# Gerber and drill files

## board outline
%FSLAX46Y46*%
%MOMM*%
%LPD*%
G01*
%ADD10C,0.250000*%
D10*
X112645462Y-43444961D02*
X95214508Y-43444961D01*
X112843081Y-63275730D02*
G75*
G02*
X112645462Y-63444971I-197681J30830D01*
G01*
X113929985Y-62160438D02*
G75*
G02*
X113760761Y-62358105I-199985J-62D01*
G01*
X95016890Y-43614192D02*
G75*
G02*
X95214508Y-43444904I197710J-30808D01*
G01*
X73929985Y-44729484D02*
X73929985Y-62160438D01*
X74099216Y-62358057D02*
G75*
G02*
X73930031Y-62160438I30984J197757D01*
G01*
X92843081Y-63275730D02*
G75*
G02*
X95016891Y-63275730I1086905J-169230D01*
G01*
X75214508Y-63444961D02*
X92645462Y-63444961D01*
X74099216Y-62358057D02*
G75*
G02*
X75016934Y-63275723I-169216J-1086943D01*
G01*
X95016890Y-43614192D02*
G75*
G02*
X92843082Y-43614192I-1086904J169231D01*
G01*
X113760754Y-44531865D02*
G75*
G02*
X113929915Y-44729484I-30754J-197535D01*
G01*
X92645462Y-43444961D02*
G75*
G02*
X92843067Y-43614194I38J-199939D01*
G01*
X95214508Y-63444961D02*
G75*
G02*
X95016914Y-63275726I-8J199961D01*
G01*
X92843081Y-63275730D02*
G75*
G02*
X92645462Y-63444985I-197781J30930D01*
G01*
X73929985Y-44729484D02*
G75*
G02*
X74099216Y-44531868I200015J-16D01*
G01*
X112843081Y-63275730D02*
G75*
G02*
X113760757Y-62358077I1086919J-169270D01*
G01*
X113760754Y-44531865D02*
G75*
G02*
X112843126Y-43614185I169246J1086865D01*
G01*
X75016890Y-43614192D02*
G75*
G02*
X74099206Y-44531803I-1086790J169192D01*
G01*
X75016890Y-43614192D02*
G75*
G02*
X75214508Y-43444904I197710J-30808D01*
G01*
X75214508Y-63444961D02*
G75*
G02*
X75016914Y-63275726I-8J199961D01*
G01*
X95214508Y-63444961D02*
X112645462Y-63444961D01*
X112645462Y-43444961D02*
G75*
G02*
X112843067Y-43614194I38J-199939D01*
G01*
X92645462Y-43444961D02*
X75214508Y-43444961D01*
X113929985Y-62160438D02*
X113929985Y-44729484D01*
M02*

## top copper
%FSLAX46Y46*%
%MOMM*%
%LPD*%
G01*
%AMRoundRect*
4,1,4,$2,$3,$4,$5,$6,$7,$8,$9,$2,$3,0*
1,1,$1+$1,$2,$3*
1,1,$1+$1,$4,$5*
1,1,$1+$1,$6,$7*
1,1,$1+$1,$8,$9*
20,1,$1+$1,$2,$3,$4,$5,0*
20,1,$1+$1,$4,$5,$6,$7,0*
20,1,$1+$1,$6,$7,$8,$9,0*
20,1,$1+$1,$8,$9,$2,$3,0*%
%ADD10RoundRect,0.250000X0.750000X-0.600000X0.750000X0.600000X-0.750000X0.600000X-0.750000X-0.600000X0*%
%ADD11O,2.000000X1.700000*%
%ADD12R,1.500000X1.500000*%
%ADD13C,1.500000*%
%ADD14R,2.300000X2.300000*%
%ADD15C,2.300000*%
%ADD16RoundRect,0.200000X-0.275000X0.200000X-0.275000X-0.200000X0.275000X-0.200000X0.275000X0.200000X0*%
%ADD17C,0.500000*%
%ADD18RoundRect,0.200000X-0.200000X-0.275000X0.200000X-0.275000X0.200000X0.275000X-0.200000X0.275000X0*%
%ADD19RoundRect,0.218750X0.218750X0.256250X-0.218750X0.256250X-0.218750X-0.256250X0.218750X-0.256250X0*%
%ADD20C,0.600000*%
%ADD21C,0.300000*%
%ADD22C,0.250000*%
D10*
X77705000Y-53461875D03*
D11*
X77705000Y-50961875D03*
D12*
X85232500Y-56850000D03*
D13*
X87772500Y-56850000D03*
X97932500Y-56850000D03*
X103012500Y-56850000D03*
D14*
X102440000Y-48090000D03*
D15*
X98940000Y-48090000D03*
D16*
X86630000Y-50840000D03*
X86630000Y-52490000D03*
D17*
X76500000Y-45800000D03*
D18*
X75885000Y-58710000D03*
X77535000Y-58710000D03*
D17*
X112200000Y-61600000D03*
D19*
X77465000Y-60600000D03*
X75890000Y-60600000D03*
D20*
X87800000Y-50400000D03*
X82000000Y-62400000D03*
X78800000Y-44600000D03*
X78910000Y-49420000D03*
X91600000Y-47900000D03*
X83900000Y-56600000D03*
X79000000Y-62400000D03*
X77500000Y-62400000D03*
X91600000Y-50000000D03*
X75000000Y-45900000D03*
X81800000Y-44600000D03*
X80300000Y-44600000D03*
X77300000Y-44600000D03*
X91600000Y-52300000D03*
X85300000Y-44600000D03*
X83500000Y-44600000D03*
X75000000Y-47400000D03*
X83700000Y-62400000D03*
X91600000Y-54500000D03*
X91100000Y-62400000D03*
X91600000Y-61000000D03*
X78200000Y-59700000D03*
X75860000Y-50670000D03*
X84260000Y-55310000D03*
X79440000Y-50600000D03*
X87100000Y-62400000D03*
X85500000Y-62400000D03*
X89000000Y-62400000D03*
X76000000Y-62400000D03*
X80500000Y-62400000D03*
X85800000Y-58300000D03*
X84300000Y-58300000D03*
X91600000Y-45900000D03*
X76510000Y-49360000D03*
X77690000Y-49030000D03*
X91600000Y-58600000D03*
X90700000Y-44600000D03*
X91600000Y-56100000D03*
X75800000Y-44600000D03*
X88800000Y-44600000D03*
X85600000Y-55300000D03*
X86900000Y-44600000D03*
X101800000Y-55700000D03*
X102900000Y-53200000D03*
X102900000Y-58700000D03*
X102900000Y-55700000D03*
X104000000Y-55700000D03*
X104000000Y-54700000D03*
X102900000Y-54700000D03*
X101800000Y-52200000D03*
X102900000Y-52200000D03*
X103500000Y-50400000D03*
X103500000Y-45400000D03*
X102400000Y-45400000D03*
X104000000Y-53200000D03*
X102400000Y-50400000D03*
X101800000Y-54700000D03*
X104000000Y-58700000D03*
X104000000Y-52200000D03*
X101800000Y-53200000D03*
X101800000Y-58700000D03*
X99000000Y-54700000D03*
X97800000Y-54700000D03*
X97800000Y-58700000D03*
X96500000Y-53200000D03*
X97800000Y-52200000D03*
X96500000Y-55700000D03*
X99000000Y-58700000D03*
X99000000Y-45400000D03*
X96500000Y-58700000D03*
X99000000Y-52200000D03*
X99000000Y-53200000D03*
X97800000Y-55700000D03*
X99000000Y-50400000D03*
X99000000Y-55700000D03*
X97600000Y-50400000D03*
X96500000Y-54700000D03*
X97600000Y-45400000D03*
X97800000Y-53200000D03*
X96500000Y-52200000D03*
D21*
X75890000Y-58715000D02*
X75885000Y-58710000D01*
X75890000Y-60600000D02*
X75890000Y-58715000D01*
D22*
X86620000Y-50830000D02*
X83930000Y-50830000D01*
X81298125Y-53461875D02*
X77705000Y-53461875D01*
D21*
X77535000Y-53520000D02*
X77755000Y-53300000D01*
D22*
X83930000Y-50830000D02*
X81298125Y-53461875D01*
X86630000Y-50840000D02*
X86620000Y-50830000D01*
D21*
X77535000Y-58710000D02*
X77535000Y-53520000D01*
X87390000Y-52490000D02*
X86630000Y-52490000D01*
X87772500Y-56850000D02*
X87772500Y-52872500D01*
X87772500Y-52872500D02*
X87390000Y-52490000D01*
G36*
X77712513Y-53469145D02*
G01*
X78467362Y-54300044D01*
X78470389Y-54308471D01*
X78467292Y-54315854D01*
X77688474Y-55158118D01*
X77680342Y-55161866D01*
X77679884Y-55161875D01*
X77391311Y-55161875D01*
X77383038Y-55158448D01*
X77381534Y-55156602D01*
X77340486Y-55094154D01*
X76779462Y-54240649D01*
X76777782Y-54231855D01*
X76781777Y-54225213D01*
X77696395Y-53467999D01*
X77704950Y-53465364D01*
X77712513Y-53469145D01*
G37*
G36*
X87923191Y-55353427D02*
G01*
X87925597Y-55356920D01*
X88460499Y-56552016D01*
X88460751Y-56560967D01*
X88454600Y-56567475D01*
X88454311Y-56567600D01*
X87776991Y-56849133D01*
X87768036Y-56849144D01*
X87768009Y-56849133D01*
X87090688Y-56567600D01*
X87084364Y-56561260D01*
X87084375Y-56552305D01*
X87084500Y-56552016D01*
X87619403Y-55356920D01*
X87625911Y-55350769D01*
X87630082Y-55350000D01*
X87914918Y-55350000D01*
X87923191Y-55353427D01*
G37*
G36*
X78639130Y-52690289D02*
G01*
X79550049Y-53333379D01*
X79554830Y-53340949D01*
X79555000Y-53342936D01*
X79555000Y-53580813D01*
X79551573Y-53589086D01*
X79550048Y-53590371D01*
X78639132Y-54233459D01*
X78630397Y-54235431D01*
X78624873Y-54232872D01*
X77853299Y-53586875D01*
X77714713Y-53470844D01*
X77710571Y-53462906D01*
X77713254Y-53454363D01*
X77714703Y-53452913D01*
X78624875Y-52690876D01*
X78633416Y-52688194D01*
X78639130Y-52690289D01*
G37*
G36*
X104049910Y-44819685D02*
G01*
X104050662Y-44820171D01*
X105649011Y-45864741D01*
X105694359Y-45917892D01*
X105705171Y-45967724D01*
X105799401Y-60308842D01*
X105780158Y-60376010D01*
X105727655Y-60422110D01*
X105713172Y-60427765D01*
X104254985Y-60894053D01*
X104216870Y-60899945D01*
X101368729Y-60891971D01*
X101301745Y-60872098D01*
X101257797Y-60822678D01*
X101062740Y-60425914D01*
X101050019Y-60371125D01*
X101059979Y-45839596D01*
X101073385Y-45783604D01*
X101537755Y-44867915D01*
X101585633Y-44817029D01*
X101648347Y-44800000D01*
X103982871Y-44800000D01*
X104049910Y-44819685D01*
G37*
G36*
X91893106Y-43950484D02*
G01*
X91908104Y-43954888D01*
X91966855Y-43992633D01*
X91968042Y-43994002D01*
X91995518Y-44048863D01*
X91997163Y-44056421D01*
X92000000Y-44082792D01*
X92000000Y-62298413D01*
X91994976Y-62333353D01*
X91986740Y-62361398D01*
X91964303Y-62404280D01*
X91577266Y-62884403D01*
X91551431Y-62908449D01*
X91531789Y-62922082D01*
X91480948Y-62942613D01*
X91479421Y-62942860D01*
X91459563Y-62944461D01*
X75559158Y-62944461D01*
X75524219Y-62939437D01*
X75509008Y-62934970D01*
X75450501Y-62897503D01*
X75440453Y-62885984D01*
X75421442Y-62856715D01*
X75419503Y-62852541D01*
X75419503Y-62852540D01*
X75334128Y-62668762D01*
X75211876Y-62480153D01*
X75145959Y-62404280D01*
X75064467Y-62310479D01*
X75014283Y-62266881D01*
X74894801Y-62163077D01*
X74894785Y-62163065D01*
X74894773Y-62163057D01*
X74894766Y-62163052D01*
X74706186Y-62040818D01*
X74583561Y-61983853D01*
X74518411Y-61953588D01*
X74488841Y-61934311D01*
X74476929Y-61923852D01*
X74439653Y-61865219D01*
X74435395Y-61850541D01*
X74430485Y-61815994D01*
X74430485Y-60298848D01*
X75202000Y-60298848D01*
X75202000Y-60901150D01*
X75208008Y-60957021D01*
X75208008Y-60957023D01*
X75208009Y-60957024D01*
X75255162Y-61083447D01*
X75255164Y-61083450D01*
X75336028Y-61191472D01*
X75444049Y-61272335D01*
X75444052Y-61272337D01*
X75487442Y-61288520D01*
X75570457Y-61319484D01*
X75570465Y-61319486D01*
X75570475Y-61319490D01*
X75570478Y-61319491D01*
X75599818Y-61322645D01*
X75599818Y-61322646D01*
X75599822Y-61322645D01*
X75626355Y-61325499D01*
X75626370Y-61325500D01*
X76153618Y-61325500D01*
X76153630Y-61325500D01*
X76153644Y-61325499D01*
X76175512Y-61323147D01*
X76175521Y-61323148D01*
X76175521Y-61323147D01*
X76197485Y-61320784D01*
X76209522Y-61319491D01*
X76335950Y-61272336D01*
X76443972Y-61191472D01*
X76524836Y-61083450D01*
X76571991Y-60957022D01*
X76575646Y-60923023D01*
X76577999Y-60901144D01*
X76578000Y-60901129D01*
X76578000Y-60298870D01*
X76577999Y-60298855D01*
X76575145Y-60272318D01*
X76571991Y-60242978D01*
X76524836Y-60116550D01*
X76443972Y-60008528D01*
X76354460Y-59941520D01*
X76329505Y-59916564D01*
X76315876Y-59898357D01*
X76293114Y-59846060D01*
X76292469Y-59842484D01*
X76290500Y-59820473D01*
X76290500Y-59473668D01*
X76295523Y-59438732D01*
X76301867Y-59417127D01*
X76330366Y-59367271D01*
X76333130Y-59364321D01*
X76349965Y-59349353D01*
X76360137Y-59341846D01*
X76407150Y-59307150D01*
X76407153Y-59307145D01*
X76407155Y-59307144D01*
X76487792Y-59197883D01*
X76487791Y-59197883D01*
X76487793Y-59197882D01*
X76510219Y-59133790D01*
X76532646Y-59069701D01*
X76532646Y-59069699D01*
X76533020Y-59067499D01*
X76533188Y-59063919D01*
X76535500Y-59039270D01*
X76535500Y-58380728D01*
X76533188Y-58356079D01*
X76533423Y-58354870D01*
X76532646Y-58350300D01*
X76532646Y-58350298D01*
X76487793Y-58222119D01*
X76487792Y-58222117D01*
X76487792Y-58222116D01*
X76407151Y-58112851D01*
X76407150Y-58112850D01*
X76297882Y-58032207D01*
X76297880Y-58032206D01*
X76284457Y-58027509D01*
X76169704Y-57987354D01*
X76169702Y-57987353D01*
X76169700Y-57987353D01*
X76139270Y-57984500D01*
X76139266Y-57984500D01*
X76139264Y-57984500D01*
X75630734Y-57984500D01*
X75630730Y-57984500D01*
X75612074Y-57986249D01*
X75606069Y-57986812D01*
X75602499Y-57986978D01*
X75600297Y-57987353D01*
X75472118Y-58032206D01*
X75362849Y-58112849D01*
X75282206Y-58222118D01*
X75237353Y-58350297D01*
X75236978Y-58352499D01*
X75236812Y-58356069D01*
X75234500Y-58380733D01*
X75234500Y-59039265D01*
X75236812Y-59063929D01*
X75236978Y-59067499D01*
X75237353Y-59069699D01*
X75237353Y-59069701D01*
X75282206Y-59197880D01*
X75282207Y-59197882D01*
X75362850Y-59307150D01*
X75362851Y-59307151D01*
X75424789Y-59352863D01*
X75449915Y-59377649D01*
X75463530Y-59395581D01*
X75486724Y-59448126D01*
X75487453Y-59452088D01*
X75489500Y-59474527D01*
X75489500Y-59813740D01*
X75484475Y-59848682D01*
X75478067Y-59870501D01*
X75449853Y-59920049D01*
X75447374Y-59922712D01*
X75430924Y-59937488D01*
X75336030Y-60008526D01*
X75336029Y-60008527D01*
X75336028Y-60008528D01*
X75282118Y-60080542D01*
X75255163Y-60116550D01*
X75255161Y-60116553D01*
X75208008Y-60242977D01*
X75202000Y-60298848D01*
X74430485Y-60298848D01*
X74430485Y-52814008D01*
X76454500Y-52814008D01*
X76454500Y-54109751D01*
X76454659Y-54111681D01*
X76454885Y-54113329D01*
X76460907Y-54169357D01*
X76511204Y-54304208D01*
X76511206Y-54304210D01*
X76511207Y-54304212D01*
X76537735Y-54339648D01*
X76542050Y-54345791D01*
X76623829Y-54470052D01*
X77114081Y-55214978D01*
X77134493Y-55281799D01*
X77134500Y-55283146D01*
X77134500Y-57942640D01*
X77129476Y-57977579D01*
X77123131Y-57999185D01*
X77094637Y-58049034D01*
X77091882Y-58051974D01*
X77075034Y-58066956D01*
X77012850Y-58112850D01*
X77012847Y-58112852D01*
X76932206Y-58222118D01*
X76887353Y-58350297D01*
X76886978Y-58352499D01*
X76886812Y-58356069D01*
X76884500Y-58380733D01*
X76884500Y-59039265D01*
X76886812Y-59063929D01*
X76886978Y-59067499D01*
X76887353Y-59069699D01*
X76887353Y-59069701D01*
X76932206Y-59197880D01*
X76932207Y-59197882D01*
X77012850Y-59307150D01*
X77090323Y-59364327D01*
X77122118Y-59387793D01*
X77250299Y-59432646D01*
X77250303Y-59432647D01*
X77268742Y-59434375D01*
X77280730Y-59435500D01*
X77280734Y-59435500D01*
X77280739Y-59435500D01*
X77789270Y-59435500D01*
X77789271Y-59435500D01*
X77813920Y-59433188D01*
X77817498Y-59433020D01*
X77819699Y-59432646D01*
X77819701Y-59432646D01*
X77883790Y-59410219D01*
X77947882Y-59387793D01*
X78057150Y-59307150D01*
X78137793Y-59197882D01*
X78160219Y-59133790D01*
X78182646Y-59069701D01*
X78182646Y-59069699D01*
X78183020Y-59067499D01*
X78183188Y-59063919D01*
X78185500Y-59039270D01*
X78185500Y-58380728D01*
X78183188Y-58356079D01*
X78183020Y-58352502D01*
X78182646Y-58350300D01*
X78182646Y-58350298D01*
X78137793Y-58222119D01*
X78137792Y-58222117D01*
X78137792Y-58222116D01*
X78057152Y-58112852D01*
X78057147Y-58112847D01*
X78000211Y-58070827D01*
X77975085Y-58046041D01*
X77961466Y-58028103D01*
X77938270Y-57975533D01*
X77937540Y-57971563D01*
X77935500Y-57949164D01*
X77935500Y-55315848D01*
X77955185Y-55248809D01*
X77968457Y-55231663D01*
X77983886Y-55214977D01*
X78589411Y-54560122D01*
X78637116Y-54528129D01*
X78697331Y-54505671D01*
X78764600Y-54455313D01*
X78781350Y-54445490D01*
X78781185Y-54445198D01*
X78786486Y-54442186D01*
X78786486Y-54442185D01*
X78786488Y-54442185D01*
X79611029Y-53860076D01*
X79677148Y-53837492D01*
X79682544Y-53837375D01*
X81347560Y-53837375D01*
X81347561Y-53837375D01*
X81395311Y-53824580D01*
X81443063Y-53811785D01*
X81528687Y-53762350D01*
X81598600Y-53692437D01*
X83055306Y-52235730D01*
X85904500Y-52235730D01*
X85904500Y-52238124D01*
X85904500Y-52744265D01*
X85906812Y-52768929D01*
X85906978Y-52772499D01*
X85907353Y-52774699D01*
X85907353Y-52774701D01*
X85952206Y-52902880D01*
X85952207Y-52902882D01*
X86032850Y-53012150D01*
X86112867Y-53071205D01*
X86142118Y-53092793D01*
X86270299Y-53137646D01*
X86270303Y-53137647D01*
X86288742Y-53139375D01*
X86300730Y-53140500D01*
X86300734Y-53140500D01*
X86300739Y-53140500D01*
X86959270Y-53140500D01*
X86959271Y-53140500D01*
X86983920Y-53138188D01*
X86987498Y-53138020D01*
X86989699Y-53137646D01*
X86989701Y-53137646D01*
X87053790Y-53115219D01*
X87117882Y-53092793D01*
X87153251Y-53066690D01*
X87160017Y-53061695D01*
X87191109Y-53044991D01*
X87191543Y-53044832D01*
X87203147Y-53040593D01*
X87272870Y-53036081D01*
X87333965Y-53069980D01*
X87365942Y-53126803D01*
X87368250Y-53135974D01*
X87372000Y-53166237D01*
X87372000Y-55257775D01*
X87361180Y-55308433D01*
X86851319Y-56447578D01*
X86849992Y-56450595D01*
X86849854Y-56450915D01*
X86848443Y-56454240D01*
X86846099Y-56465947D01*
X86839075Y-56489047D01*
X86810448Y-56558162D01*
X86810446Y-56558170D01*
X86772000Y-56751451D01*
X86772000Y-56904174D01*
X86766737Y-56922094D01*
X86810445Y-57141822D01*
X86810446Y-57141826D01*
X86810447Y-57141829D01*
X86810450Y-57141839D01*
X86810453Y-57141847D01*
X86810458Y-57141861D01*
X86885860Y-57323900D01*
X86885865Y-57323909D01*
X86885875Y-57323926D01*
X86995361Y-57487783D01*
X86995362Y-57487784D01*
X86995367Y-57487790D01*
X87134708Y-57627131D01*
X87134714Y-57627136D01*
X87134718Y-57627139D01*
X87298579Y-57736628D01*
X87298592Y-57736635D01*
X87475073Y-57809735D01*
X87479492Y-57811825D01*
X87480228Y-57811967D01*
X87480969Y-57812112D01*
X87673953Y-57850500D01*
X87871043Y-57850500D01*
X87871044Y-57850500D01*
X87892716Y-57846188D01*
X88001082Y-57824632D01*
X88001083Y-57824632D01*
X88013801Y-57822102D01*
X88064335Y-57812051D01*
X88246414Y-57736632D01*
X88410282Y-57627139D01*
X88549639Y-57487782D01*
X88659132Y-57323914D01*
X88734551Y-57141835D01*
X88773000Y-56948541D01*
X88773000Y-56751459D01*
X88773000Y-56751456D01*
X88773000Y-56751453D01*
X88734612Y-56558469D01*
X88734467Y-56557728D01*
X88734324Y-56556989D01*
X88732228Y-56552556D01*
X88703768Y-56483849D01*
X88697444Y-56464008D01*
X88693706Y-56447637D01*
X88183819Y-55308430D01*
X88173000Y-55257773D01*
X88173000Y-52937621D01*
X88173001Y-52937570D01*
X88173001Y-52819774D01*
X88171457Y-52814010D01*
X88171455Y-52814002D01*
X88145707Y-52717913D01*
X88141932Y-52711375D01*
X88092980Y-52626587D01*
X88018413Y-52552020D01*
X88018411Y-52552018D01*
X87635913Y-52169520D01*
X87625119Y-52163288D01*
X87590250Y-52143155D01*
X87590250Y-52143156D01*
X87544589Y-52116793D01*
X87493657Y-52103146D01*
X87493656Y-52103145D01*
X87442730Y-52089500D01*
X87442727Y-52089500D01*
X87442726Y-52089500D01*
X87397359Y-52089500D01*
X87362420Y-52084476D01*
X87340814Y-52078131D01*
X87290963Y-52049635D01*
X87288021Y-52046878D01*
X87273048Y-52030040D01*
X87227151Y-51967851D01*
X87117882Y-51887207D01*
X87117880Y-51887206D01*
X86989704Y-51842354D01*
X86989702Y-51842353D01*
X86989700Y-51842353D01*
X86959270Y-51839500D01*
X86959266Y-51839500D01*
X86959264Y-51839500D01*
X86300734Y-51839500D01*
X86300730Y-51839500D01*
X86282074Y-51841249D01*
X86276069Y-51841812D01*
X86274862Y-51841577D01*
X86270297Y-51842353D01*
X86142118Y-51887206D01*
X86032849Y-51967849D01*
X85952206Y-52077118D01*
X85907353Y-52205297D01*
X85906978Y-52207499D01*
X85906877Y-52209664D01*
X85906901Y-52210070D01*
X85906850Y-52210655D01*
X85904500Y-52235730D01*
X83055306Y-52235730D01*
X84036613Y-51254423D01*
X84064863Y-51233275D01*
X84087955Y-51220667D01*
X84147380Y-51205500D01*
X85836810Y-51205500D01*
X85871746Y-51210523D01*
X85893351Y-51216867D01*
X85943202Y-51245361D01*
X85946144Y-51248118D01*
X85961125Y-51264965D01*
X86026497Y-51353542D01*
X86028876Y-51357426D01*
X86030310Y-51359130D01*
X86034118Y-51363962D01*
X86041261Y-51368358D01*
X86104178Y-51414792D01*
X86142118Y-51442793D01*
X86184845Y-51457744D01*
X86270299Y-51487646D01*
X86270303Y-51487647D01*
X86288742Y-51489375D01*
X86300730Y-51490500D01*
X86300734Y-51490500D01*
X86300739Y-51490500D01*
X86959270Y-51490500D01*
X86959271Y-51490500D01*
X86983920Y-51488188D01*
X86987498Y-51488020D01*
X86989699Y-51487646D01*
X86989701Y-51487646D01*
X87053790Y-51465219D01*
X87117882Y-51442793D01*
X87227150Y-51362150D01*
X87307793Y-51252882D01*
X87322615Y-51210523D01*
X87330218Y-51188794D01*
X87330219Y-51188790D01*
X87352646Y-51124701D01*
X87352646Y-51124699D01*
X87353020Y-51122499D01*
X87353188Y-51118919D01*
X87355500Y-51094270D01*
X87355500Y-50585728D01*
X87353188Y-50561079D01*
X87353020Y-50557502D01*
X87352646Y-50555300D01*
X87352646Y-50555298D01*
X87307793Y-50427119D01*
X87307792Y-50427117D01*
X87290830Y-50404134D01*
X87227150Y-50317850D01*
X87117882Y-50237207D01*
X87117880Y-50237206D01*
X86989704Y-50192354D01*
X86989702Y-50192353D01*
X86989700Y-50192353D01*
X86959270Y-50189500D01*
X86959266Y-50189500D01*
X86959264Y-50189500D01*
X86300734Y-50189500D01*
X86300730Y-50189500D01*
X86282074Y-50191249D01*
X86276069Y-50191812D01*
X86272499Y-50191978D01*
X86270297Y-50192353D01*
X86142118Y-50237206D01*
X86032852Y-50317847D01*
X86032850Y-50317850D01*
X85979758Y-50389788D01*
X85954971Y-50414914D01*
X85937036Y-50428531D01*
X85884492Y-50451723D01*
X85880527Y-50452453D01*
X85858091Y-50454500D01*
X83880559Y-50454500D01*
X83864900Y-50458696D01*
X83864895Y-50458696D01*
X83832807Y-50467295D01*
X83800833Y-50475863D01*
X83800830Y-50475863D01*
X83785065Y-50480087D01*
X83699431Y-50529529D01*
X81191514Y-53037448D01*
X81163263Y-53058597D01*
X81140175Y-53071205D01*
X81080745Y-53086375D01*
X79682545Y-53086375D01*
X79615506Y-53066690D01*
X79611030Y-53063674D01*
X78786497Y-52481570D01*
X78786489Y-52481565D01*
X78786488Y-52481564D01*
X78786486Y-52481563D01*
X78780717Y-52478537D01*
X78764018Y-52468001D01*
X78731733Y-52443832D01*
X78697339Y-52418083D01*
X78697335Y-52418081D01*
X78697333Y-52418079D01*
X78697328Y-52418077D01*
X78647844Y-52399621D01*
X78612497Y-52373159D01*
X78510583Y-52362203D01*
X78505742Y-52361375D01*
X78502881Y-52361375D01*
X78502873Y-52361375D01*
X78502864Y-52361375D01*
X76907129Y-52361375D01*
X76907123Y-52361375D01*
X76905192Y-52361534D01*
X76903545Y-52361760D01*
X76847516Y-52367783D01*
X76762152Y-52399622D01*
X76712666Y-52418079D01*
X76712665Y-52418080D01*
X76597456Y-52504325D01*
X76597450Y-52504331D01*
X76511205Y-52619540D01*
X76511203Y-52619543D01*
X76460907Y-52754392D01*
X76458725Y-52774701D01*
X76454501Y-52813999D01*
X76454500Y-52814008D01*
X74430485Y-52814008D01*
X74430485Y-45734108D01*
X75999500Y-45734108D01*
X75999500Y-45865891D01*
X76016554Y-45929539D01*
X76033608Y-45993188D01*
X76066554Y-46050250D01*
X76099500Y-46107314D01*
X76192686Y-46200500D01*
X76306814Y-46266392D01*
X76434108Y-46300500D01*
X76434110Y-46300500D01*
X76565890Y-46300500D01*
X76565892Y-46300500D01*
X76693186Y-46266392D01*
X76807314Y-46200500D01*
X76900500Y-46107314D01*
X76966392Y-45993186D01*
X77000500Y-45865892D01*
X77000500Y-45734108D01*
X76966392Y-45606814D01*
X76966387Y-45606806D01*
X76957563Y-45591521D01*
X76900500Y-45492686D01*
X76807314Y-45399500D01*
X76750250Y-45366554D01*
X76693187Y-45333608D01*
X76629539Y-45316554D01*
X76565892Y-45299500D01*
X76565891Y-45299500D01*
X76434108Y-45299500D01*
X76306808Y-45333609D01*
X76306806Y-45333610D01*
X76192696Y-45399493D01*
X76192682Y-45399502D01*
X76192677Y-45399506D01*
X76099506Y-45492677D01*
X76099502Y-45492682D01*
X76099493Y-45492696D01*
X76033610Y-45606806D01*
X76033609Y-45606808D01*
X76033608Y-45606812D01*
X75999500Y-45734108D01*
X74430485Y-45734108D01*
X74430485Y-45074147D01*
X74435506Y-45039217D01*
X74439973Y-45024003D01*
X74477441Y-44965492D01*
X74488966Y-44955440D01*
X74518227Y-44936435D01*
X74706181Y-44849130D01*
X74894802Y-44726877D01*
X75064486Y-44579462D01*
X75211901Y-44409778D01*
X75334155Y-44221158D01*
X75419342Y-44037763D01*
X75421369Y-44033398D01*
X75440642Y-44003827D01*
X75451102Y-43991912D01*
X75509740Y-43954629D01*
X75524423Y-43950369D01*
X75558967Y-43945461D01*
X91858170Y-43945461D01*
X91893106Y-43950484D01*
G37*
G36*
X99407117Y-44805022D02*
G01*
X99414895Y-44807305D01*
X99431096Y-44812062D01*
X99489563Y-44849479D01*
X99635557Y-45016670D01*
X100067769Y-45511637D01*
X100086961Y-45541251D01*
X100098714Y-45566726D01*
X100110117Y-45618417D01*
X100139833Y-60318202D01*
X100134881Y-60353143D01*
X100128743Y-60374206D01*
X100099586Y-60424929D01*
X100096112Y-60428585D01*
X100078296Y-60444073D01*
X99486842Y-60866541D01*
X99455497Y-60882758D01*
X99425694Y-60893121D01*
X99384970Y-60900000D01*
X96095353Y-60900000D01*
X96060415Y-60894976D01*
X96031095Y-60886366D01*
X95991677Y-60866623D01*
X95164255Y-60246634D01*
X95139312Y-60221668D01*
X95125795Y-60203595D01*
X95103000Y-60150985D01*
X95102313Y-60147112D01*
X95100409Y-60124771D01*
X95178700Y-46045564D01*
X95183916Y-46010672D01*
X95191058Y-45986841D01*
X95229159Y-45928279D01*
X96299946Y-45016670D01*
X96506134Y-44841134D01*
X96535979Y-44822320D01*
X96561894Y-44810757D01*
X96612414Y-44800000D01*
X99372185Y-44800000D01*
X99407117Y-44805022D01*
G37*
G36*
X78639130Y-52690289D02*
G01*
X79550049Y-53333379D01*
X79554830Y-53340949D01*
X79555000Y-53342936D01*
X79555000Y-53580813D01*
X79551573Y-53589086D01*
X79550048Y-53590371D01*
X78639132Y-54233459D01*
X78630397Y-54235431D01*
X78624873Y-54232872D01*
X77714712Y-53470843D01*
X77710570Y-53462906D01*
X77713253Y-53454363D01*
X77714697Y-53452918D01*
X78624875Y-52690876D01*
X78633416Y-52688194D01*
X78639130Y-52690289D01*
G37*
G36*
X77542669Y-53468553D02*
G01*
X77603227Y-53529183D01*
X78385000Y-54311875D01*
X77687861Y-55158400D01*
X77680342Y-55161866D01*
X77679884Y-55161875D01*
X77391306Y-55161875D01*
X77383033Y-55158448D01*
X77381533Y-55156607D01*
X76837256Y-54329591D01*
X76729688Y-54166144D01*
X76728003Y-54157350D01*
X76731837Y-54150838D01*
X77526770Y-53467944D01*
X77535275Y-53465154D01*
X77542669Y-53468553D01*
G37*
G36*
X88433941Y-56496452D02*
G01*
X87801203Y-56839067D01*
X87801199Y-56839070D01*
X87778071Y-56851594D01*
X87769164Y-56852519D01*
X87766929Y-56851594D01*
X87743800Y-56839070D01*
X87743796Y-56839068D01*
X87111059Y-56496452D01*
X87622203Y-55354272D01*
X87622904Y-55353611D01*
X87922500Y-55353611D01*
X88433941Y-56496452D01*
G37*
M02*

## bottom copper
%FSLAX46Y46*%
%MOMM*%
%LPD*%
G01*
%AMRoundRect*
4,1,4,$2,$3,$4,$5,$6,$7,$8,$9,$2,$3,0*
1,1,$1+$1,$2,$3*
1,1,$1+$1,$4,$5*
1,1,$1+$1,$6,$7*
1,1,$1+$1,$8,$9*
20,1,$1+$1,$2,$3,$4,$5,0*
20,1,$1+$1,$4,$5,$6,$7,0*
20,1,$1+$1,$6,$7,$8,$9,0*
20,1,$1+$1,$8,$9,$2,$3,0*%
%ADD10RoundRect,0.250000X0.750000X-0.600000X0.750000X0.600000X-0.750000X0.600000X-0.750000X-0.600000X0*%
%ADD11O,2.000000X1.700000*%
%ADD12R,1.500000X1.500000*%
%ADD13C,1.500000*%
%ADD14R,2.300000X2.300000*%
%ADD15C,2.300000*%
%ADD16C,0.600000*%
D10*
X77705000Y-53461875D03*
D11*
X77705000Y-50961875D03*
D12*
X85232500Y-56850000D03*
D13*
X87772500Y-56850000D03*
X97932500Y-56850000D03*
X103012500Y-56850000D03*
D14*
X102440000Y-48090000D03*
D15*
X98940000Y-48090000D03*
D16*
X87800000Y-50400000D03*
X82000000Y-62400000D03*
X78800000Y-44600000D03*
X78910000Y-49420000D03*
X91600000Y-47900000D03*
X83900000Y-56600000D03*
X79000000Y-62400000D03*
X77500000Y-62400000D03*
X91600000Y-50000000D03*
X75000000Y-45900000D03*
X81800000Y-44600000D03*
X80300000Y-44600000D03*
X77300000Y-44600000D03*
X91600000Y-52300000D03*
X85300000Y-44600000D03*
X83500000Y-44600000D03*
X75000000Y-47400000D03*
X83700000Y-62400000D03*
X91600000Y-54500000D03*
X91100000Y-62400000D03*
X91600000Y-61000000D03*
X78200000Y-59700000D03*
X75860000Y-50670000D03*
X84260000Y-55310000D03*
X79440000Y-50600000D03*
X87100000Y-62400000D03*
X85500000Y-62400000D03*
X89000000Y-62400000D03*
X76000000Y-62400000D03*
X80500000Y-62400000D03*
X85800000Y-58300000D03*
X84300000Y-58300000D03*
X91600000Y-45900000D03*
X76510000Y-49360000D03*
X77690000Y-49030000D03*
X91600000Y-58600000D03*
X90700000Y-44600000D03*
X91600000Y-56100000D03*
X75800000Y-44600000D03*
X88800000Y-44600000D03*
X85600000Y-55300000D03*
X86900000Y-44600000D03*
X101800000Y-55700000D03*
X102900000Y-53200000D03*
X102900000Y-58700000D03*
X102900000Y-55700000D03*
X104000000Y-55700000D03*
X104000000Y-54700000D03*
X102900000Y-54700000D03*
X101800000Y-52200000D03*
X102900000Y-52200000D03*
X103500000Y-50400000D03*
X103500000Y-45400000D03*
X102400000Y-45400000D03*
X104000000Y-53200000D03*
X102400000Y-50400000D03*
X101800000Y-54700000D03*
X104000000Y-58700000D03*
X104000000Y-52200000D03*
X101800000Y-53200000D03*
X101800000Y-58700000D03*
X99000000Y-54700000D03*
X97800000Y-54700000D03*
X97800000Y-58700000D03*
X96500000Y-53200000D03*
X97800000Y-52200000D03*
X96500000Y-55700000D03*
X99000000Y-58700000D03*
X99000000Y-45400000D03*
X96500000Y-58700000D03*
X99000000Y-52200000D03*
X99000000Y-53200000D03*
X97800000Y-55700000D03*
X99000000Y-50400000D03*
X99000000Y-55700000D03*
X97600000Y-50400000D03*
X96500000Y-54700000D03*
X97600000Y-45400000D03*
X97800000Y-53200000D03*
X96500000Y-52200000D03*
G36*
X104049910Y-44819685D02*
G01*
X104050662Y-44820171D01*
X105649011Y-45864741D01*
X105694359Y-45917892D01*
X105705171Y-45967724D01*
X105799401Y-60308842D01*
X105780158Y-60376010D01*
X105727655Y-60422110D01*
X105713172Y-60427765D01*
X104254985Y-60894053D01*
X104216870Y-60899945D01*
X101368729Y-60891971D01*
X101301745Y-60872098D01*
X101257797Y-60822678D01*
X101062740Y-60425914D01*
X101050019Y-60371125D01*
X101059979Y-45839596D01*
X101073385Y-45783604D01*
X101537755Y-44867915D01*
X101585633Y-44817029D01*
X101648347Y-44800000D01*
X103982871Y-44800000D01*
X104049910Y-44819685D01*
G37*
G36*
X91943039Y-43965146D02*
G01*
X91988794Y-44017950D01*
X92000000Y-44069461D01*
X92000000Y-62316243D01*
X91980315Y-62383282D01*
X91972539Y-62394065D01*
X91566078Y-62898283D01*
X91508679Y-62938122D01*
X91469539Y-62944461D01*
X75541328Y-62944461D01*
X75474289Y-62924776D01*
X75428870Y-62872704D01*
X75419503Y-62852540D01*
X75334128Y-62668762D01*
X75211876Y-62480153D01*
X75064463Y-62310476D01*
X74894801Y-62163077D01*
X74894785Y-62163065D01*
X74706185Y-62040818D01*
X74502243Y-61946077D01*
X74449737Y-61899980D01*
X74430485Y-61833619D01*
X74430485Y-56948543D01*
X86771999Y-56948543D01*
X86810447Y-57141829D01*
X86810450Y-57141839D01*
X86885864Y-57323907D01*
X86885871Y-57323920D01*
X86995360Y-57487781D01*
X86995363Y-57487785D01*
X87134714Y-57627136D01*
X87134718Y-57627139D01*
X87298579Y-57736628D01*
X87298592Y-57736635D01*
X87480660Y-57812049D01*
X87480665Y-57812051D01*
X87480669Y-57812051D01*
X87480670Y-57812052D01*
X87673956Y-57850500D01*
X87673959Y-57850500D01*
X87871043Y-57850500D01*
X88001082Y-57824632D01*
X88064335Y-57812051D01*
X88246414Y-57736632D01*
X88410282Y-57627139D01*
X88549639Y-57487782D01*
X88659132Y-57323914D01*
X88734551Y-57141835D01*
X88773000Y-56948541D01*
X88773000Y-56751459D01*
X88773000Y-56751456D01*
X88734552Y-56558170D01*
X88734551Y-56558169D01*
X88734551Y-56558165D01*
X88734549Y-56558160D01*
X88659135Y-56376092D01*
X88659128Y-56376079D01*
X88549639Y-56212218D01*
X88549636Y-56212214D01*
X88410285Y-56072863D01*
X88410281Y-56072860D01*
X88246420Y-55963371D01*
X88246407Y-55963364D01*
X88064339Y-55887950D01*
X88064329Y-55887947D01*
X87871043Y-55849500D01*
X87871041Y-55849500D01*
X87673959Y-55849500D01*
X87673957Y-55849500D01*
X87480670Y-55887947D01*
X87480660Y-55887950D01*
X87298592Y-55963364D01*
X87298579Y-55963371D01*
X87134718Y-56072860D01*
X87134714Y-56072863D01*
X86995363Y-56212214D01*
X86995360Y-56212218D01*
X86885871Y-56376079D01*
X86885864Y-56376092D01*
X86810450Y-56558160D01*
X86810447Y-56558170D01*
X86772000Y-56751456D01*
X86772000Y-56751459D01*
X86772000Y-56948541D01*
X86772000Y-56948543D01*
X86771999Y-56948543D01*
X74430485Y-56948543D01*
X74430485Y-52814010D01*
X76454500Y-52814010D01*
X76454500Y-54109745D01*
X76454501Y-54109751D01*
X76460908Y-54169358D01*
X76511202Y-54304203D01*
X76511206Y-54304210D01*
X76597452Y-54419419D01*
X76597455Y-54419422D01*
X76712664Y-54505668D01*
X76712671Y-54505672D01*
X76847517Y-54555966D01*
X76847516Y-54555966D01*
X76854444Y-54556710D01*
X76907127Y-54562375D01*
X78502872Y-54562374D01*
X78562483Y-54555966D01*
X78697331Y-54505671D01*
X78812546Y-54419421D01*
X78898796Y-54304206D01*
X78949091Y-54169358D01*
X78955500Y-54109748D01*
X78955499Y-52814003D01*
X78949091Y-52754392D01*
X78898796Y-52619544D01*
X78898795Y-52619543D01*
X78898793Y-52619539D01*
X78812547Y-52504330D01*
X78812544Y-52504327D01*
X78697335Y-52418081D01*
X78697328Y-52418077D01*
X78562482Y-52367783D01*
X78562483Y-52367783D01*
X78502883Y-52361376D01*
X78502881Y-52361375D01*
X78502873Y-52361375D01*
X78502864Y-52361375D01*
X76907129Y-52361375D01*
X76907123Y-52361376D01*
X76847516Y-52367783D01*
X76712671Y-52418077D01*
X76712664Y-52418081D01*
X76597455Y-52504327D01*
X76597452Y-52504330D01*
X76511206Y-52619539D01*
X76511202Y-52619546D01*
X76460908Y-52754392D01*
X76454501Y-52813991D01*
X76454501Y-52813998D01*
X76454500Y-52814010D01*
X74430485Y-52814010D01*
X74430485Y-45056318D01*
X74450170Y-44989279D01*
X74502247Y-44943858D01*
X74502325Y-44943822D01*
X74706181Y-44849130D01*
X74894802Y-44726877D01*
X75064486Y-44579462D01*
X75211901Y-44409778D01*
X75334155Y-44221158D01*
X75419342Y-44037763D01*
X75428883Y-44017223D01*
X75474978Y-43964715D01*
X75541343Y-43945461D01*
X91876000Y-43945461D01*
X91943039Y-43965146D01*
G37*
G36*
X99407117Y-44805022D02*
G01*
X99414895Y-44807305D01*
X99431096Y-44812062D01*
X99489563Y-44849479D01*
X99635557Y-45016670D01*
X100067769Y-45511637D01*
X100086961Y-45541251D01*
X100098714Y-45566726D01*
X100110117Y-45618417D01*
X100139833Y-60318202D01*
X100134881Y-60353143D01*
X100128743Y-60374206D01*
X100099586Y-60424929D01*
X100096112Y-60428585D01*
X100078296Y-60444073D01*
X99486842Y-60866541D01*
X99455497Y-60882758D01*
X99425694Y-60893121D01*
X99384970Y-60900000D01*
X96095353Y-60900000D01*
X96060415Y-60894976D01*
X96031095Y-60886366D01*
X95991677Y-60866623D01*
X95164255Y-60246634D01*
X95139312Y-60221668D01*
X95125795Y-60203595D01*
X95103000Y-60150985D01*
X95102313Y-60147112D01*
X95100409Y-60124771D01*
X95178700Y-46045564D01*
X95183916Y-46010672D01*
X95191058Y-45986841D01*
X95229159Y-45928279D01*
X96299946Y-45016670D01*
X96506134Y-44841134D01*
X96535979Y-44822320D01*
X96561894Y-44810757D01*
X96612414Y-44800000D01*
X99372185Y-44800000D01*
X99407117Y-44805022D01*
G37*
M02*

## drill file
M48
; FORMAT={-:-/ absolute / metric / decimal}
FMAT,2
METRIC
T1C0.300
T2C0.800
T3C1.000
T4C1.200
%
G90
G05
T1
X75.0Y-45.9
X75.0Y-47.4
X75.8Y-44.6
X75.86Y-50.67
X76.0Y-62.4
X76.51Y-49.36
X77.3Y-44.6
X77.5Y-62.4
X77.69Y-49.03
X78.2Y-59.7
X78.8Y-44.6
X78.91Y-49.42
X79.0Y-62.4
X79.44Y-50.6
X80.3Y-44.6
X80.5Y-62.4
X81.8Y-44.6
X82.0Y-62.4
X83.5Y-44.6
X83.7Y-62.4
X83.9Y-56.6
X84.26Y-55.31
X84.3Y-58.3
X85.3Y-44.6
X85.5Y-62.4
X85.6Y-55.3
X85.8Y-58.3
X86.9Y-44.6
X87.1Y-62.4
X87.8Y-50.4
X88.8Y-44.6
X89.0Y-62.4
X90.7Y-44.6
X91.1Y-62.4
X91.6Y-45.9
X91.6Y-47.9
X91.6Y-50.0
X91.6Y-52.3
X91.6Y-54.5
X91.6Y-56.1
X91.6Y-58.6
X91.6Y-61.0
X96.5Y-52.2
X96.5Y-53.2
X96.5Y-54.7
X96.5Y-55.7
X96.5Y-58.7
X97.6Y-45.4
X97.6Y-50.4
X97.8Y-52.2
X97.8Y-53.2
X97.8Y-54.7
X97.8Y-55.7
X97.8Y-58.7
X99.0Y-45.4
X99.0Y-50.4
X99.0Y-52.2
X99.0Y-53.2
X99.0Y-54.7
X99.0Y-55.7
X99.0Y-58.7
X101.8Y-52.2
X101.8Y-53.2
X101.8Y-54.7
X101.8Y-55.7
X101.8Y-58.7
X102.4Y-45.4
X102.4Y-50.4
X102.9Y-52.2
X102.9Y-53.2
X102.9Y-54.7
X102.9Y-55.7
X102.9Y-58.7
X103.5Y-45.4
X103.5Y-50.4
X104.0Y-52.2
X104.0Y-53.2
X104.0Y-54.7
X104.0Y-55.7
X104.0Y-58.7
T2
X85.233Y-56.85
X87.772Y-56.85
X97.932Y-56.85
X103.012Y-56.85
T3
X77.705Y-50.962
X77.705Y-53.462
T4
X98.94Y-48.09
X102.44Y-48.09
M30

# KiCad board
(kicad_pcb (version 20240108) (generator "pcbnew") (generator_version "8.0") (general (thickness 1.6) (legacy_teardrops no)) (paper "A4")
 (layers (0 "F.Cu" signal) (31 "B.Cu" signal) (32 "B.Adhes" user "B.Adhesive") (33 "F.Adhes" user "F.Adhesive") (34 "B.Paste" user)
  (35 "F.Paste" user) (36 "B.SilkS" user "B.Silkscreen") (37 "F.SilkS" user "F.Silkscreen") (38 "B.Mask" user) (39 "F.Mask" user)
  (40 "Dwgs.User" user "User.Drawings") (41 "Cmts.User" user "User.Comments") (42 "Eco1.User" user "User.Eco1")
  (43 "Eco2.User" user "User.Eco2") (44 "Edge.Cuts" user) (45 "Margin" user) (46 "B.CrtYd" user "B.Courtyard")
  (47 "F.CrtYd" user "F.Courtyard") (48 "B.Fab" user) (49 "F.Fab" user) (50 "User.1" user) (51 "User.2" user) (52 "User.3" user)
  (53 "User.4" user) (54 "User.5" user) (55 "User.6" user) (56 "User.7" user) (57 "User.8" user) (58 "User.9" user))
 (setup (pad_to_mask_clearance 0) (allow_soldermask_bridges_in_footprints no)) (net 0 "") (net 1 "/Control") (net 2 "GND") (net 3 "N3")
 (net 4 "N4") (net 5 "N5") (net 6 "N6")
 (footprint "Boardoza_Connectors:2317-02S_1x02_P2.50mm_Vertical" (layer "F.Cu") (at 77.655 52.301875 90)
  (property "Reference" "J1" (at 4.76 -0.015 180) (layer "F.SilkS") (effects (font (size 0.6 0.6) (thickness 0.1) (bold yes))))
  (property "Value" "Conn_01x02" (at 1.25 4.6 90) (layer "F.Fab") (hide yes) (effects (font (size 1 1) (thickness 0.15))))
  (pad "1" thru_hole roundrect (at -1.16 0.05 90) (size 1.7 2) (drill 1) (layers "*.Cu" "*.Mask") (remove_unused_layers no)
   (roundrect_rratio 0.1470588235) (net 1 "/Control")
   (teardrops (best_length_ratio 0.5) (max_length 1) (best_width_ratio 1) (max_width 2) (curve_points 0) (filter_ratio 0.9) (enabled yes)
    (allow_two_segments yes) (prefer_zone_connections yes)))
  (pad "2" thru_hole oval (at 1.34 0.05 90) (size 1.7 2) (drill 1) (layers "*.Cu" "*.Mask") (remove_unused_layers no) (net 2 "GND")
   (teardrops (best_length_ratio 0.5) (max_length 1) (best_width_ratio 1) (max_width 2) (curve_points 0) (filter_ratio 0.9) (enabled yes)
    (allow_two_segments yes) (prefer_zone_connections yes))))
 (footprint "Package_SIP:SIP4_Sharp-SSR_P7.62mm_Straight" (layer "F.Cu") (at 103.0125 57.85 180)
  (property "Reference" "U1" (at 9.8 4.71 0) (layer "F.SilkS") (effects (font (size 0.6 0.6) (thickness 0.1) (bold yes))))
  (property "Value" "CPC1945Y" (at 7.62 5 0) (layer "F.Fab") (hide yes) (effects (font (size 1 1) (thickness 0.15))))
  (pad "1" thru_hole rect (at 17.78 1 180) (size 1.5 1.5) (drill 0.8) (layers "*.Cu" "*.Mask") (remove_unused_layers no) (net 2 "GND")
   (teardrops (best_length_ratio 0.5) (max_length 1) (best_width_ratio 1) (max_width 2) (curve_points 0) (filter_ratio 0.9) (enabled yes)
    (allow_two_segments yes) (prefer_zone_connections yes)))
  (pad "2" thru_hole circle (at 15.24 1 180) (size 1.5 1.5) (drill 0.8) (layers "*.Cu" "*.Mask") (remove_unused_layers no) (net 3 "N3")
   (teardrops (best_length_ratio 0.5) (max_length 1) (best_width_ratio 1) (max_width 2) (curve_points 0) (filter_ratio 0.9) (enabled yes)
    (allow_two_segments yes) (prefer_zone_connections yes)))
  (pad "6" thru_hole circle (at 5.08 1 180) (size 1.5 1.5) (drill 0.8) (layers "*.Cu" "*.Mask") (remove_unused_layers no) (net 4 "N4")
   (teardrops (best_length_ratio 0.5) (max_length 1) (best_width_ratio 1) (max_width 2) (curve_points 0) (filter_ratio 0.9) (enabled yes)
    (allow_two_segments yes) (prefer_zone_connections yes)))
  (pad "8" thru_hole circle (at 0 1 180) (size 1.5 1.5) (drill 0.8) (layers "*.Cu" "*.Mask") (remove_unused_layers no) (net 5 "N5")
   (teardrops (best_length_ratio 0.5) (max_length 1) (best_width_ratio 1) (max_width 2) (curve_points 0) (filter_ratio 0.9) (enabled yes)
    (allow_two_segments yes) (prefer_zone_connections yes))))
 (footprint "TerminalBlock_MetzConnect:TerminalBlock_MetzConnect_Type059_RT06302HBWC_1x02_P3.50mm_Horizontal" (layer "F.Cu")
  (at 102.44 48.09 180)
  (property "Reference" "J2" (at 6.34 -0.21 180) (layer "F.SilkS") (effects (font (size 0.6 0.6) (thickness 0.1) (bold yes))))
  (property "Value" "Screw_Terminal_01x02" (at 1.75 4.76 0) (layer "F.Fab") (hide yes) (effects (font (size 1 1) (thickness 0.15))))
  (pad "1" thru_hole rect (at 0 0 180) (size 2.3 2.3) (drill 1.2) (layers "*.Cu" "*.Mask") (remove_unused_layers no) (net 5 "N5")
   (teardrops (best_length_ratio 0.5) (max_length 1) (best_width_ratio 1) (max_width 2) (curve_points 0) (filter_ratio 0.9) (enabled yes)
    (allow_two_segments yes) (prefer_zone_connections yes)))
  (pad "2" thru_hole circle (at 3.5 0 180) (size 2.3 2.3) (drill 1.2) (layers "*.Cu" "*.Mask") (remove_unused_layers no) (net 4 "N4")
   (teardrops (best_length_ratio 0.5) (max_length 1) (best_width_ratio 1) (max_width 2) (curve_points 0) (filter_ratio 0.9) (enabled yes)
    (allow_two_segments yes) (prefer_zone_connections yes))))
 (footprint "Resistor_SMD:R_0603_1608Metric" (layer "F.Cu") (at 86.63 51.665 -90)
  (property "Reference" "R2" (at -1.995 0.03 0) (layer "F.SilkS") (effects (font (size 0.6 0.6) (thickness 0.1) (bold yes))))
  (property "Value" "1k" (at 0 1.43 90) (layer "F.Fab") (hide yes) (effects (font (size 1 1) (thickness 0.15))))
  (pad "1" smd roundrect (at -0.825 0 270) (size 0.8 0.95) (layers "F.Cu" "F.Paste" "F.Mask") (roundrect_rratio 0.25) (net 1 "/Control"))
  (pad "2" smd roundrect (at 0.825 0 270) (size 0.8 0.95) (layers "F.Cu" "F.Paste" "F.Mask") (roundrect_rratio 0.25) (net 3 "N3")))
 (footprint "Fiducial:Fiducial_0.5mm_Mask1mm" (layer "F.Cu") (at 76.5 45.8)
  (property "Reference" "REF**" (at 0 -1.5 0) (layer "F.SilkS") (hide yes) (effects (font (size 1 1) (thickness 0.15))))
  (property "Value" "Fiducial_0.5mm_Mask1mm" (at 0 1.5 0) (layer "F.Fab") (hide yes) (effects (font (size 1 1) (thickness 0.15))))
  (pad "" smd circle (at 0 0) (size 0.5 0.5) (layers "F.Cu" "F.Mask") (solder_mask_margin 0.25) (clearance 0.25)))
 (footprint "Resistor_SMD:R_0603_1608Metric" (layer "F.Cu") (at 76.71 58.71)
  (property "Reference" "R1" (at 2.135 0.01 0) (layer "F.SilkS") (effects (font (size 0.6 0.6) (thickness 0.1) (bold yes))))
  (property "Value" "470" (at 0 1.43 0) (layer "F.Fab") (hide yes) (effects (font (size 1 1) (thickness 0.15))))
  (pad "1" smd roundrect (at -0.825 0) (size 0.8 0.95) (layers "F.Cu" "F.Paste" "F.Mask") (roundrect_rratio 0.25) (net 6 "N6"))
  (pad "2" smd roundrect (at 0.825 0) (size 0.8 0.95) (layers "F.Cu" "F.Paste" "F.Mask") (roundrect_rratio 0.25) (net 1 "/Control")))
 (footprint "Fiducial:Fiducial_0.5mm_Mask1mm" (layer "F.Cu") (at 112.2 61.6)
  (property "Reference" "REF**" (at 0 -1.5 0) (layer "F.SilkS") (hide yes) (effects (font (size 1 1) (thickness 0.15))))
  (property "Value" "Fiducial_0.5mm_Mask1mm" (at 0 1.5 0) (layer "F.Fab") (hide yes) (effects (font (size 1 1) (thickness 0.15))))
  (pad "" smd circle (at 0 0) (size 0.5 0.5) (layers "F.Cu" "F.Mask") (solder_mask_margin 0.25) (clearance 0.25)))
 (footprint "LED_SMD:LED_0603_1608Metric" (layer "F.Cu") (at 76.6775 60.6 180)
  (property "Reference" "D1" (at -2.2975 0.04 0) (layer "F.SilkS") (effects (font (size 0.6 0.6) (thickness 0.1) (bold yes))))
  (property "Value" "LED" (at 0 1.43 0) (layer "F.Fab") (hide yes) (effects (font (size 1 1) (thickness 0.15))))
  (pad "1" smd roundrect (at -0.7875 0 180) (size 0.875 0.95) (layers "F.Cu" "F.Paste" "F.Mask") (roundrect_rratio 0.25) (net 2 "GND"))
  (pad "2" smd roundrect (at 0.7875 0 180) (size 0.875 0.95) (layers "F.Cu" "F.Paste" "F.Mask") (roundrect_rratio 0.25) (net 6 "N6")))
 (gr_line (start 112.645462 43.444961) (end 95.214508 43.444961) (stroke (width 0.25) (type solid)) (layer "Edge.Cuts"))
 (gr_arc (start 112.843081 63.27573) (mid 112.775541 63.39686) (end 112.645462 63.444961) (stroke (width 0.25) (type solid))
  (layer "Edge.Cuts"))
 (gr_arc (start 113.929985 62.160438) (mid 113.881906 62.290535) (end 113.760754 62.358057) (stroke (width 0.25) (type solid))
  (layer "Edge.Cuts"))
 (gr_arc (start 95.01689 43.614192) (mid 95.084437 43.493071) (end 95.214508 43.444961) (stroke (width 0.25) (type solid))
  (layer "Edge.Cuts"))
 (gr_line (start 73.929985 44.729484) (end 73.929985 62.160438) (stroke (width 0.25) (type solid)) (layer "Edge.Cuts"))
 (gr_arc (start 74.099216 62.358057) (mid 73.978117 62.29049) (end 73.929985 62.160438) (stroke (width 0.25) (type solid))
  (layer "Edge.Cuts"))
 (gr_arc (start 92.843081 63.27573) (mid 93.929985 62.34496) (end 95.01689 63.27573) (stroke (width 0.25) (type solid)) (layer "Edge.Cuts"))
 (gr_line (start 75.214508 63.444961) (end 92.645462 63.444961) (stroke (width 0.25) (type solid)) (layer "Edge.Cuts"))
 (gr_arc (start 74.099216 62.358057) (mid 74.707796 62.66715) (end 75.01689 63.27573) (stroke (width 0.25) (type solid)) (layer "Edge.Cuts"))
 (gr_arc (start 95.01689 43.614192) (mid 93.929986 44.544961) (end 92.843081 43.614192) (stroke (width 0.25) (type solid))
  (layer "Edge.Cuts"))
 (gr_arc (start 113.760754 44.531865) (mid 113.881907 44.599386) (end 113.929985 44.729484) (stroke (width 0.25) (type solid))
  (layer "Edge.Cuts"))
 (gr_arc (start 92.645462 43.444961) (mid 92.775557 43.493043) (end 92.843081 43.614192) (stroke (width 0.25) (type solid))
  (layer "Edge.Cuts"))
 (gr_arc (start 95.214508 63.444961) (mid 95.084422 63.396869) (end 95.01689 63.27573) (stroke (width 0.25) (type solid))
  (layer "Edge.Cuts"))
 (gr_arc (start 92.843081 63.27573) (mid 92.775518 63.396834) (end 92.645462 63.444961) (stroke (width 0.25) (type solid))
  (layer "Edge.Cuts"))
 (gr_arc (start 73.929985 44.729484) (mid 73.978079 44.5994) (end 74.099216 44.531865) (stroke (width 0.25) (type solid))
  (layer "Edge.Cuts"))
 (gr_arc (start 112.843081 63.27573) (mid 113.15218 62.667156) (end 113.760754 62.358057) (stroke (width 0.25) (type solid))
  (layer "Edge.Cuts"))
 (gr_arc (start 113.760754 44.531865) (mid 113.152162 44.222784) (end 112.843081 43.614192) (stroke (width 0.25) (type solid))
  (layer "Edge.Cuts"))
 (gr_arc (start 75.01689 43.614192) (mid 74.707816 44.222791) (end 74.099216 44.531865) (stroke (width 0.25) (type solid))
  (layer "Edge.Cuts"))
 (gr_arc (start 75.01689 43.614192) (mid 75.084437 43.493071) (end 75.214508 43.444961) (stroke (width 0.25) (type solid))
  (layer "Edge.Cuts"))
 (gr_arc (start 75.214508 63.444961) (mid 75.084422 63.396869) (end 75.01689 63.27573) (stroke (width 0.25) (type solid))
  (layer "Edge.Cuts"))
 (gr_line (start 95.214508 63.444961) (end 112.645462 63.444961) (stroke (width 0.25) (type solid)) (layer "Edge.Cuts"))
 (gr_arc (start 112.645462 43.444961) (mid 112.775557 43.493043) (end 112.843081 43.614192) (stroke (width 0.25) (type solid))
  (layer "Edge.Cuts"))
 (gr_line (start 92.645462 43.444961) (end 75.214508 43.444961) (stroke (width 0.25) (type solid)) (layer "Edge.Cuts"))
 (gr_line (start 113.929985 62.160438) (end 113.929985 44.729484) (stroke (width 0.25) (type solid)) (layer "Edge.Cuts"))
 (via (at 87.8 50.4) (size 0.6) (drill 0.3) (layers "F.Cu" "B.Cu") (free yes) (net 2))
 (via (at 82 62.4) (size 0.6) (drill 0.3) (layers "F.Cu" "B.Cu") (free yes) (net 2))
 (via (at 78.8 44.6) (size 0.6) (drill 0.3) (layers "F.Cu" "B.Cu") (free yes) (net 2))
 (via (at 78.91 49.42) (size 0.6) (drill 0.3) (layers "F.Cu" "B.Cu") (free yes) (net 2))
 (via (at 91.6 47.9) (size 0.6) (drill 0.3) (layers "F.Cu" "B.Cu") (free yes) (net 2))
 (via (at 83.9 56.6) (size 0.6) (drill 0.3) (layers "F.Cu" "B.Cu") (free yes) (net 2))
 (via (at 79 62.4) (size 0.6) (drill 0.3) (layers "F.Cu" "B.Cu") (free yes) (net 2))
 (via (at 77.5 62.4) (size 0.6) (drill 0.3) (layers "F.Cu" "B.Cu") (free yes) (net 2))
 (via (at 91.6 50) (size 0.6) (drill 0.3) (layers "F.Cu" "B.Cu") (free yes) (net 2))
 (via (at 75 45.9) (size 0.6) (drill 0.3) (layers "F.Cu" "B.Cu") (free yes) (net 2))
 (via (at 81.8 44.6) (size 0.6) (drill 0.3) (layers "F.Cu" "B.Cu") (free yes) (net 2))
 (via (at 80.3 44.6) (size 0.6) (drill 0.3) (layers "F.Cu" "B.Cu") (free yes) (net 2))
 (via (at 77.3 44.6) (size 0.6) (drill 0.3) (layers "F.Cu" "B.Cu") (free yes) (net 2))
 (via (at 91.6 52.3) (size 0.6) (drill 0.3) (layers "F.Cu" "B.Cu") (free yes) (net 2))
 (via (at 85.3 44.6) (size 0.6) (drill 0.3) (layers "F.Cu" "B.Cu") (free yes) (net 2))
 (via (at 83.5 44.6) (size 0.6) (drill 0.3) (layers "F.Cu" "B.Cu") (free yes) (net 2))
 (via (at 75 47.4) (size 0.6) (drill 0.3) (layers "F.Cu" "B.Cu") (free yes) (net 2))
 (via (at 83.7 62.4) (size 0.6) (drill 0.3) (layers "F.Cu" "B.Cu") (free yes) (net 2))
 (via (at 91.6 54.5) (size 0.6) (drill 0.3) (layers "F.Cu" "B.Cu") (free yes) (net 2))
 (via (at 91.1 62.4) (size 0.6) (drill 0.3) (layers "F.Cu" "B.Cu") (free yes) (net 2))
 (via (at 91.6 61) (size 0.6) (drill 0.3) (layers "F.Cu" "B.Cu") (free yes) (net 2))
 (via (at 78.2 59.7) (size 0.6) (drill 0.3) (layers "F.Cu" "B.Cu") (free yes) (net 2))
 (via (at 75.86 50.67) (size 0.6) (drill 0.3) (layers "F.Cu" "B.Cu") (free yes) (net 2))
 (via (at 84.26 55.31) (size 0.6) (drill 0.3) (layers "F.Cu" "B.Cu") (free yes) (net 2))
 (via (at 79.44 50.6) (size 0.6) (drill 0.3) (layers "F.Cu" "B.Cu") (free yes) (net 2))
 (via (at 87.1 62.4) (size 0.6) (drill 0.3) (layers "F.Cu" "B.Cu") (free yes) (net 2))
 (via (at 85.5 62.4) (size 0.6) (drill 0.3) (layers "F.Cu" "B.Cu") (free yes) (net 2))
 (via (at 89 62.4) (size 0.6) (drill 0.3) (layers "F.Cu" "B.Cu") (free yes) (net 2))
 (via (at 76 62.4) (size 0.6) (drill 0.3) (layers "F.Cu" "B.Cu") (free yes) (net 2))
 (via (at 80.5 62.4) (size 0.6) (drill 0.3) (layers "F.Cu" "B.Cu") (free yes) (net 2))
 (via (at 85.8 58.3) (size 0.6) (drill 0.3) (layers "F.Cu" "B.Cu") (free yes) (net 2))
 (via (at 84.3 58.3) (size 0.6) (drill 0.3) (layers "F.Cu" "B.Cu") (free yes) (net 2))
 (via (at 91.6 45.9) (size 0.6) (drill 0.3) (layers "F.Cu" "B.Cu") (free yes) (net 2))
 (via (at 76.51 49.36) (size 0.6) (drill 0.3) (layers "F.Cu" "B.Cu") (free yes) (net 2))
 (via (at 77.69 49.03) (size 0.6) (drill 0.3) (layers "F.Cu" "B.Cu") (free yes) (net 2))
 (via (at 91.6 58.6) (size 0.6) (drill 0.3) (layers "F.Cu" "B.Cu") (free yes) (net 2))
 (via (at 90.7 44.6) (size 0.6) (drill 0.3) (layers "F.Cu" "B.Cu") (free yes) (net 2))
 (via (at 91.6 56.1) (size 0.6) (drill 0.3) (layers "F.Cu" "B.Cu") (free yes) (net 2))
 (via (at 75.8 44.6) (size 0.6) (drill 0.3) (layers "F.Cu" "B.Cu") (free yes) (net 2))
 (via (at 88.8 44.6) (size 0.6) (drill 0.3) (layers "F.Cu" "B.Cu") (free yes) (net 2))
 (via (at 85.6 55.3) (size 0.6) (drill 0.3) (layers "F.Cu" "B.Cu") (free yes) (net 2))
 (via (at 86.9 44.6) (size 0.6) (drill 0.3) (layers "F.Cu" "B.Cu") (free yes) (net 2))
 (segment (start 75.89 58.715) (end 75.885 58.71) (width 0.3) (layer "F.Cu") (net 6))
 (segment (start 75.89 60.6) (end 75.89 58.715) (width 0.3) (layer "F.Cu") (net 6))
 (segment (start 86.62 50.83) (end 83.93 50.83) (width 0.25) (layer "F.Cu") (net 1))
 (segment (start 81.298125 53.461875) (end 77.705 53.461875) (width 0.25) (layer "F.Cu") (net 1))
 (segment (start 77.535 53.52) (end 77.755 53.3) (width 0.3) (layer "F.Cu") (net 1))
 (segment (start 83.93 50.83) (end 81.298125 53.461875) (width 0.25) (layer "F.Cu") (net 1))
 (segment (start 86.63 50.84) (end 86.62 50.83) (width 0.25) (layer "F.Cu") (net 1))
 (segment (start 77.535 58.71) (end 77.535 53.52) (width 0.3) (layer "F.Cu") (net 1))
 (via (at 101.8 55.7) (size 0.6) (drill 0.3) (layers "F.Cu" "B.Cu") (free yes) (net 5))
 (via (at 102.9 53.2) (size 0.6) (drill 0.3) (layers "F.Cu" "B.Cu") (free yes) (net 5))
 (via (at 102.9 58.7) (size 0.6) (drill 0.3) (layers "F.Cu" "B.Cu") (free yes) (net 5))
 (via (at 102.9 55.7) (size 0.6) (drill 0.3) (layers "F.Cu" "B.Cu") (free yes) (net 5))
 (via (at 104 55.7) (size 0.6) (drill 0.3) (layers "F.Cu" "B.Cu") (free yes) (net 5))
 (via (at 104 54.7) (size 0.6) (drill 0.3) (layers "F.Cu" "B.Cu") (free yes) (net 5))
 (via (at 102.9 54.7) (size 0.6) (drill 0.3) (layers "F.Cu" "B.Cu") (free yes) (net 5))
 (via (at 101.8 52.2) (size 0.6) (drill 0.3) (layers "F.Cu" "B.Cu") (free yes) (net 5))
 (via (at 102.9 52.2) (size 0.6) (drill 0.3) (layers "F.Cu" "B.Cu") (free yes) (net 5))
 (via (at 103.5 50.4) (size 0.6) (drill 0.3) (layers "F.Cu" "B.Cu") (free yes) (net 5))
 (via (at 103.5 45.4) (size 0.6) (drill 0.3) (layers "F.Cu" "B.Cu") (free yes) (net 5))
 (via (at 102.4 45.4) (size 0.6) (drill 0.3) (layers "F.Cu" "B.Cu") (free yes) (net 5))
 (via (at 104 53.2) (size 0.6) (drill 0.3) (layers "F.Cu" "B.Cu") (free yes) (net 5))
 (via (at 102.4 50.4) (size 0.6) (drill 0.3) (layers "F.Cu" "B.Cu") (free yes) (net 5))
 (via (at 101.8 54.7) (size 0.6) (drill 0.3) (layers "F.Cu" "B.Cu") (free yes) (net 5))
 (via (at 104 58.7) (size 0.6) (drill 0.3) (layers "F.Cu" "B.Cu") (free yes) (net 5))
 (via (at 104 52.2) (size 0.6) (drill 0.3) (layers "F.Cu" "B.Cu") (free yes) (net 5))
 (via (at 101.8 53.2) (size 0.6) (drill 0.3) (layers "F.Cu" "B.Cu") (free yes) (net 5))
 (via (at 101.8 58.7) (size 0.6) (drill 0.3) (layers "F.Cu" "B.Cu") (free yes) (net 5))
 (via (at 99 54.7) (size 0.6) (drill 0.3) (layers "F.Cu" "B.Cu") (free yes) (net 4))
 (via (at 97.8 54.7) (size 0.6) (drill 0.3) (layers "F.Cu" "B.Cu") (free yes) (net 4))
 (via (at 97.8 58.7) (size 0.6) (drill 0.3) (layers "F.Cu" "B.Cu") (free yes) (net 4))
 (via (at 96.5 53.2) (size 0.6) (drill 0.3) (layers "F.Cu" "B.Cu") (free yes) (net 4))
 (via (at 97.8 52.2) (size 0.6) (drill 0.3) (layers "F.Cu" "B.Cu") (free yes) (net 4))
 (via (at 96.5 55.7) (size 0.6) (drill 0.3) (layers "F.Cu" "B.Cu") (free yes) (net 4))
 (via (at 99 58.7) (size 0.6) (drill 0.3) (layers "F.Cu" "B.Cu") (free yes) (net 4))
 (via (at 99 45.4) (size 0.6) (drill 0.3) (layers "F.Cu" "B.Cu") (free yes) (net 4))
 (via (at 96.5 58.7) (size 0.6) (drill 0.3) (layers "F.Cu" "B.Cu") (free yes) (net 4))
 (via (at 99 52.2) (size 0.6) (drill 0.3) (layers "F.Cu" "B.Cu") (free yes) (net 4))
 (via (at 99 53.2) (size 0.6) (drill 0.3) (layers "F.Cu" "B.Cu") (free yes) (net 4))
 (via (at 97.8 55.7) (size 0.6) (drill 0.3) (layers "F.Cu" "B.Cu") (free yes) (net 4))
 (via (at 99 50.4) (size 0.6) (drill 0.3) (layers "F.Cu" "B.Cu") (free yes) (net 4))
 (via (at 99 55.7) (size 0.6) (drill 0.3) (layers "F.Cu" "B.Cu") (free yes) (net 4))
 (via (at 97.6 50.4) (size 0.6) (drill 0.3) (layers "F.Cu" "B.Cu") (free yes) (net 4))
 (via (at 96.5 54.7) (size 0.6) (drill 0.3) (layers "F.Cu" "B.Cu") (free yes) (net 4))
 (via (at 97.6 45.4) (size 0.6) (drill 0.3) (layers "F.Cu" "B.Cu") (free yes) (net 4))
 (via (at 97.8 53.2) (size 0.6) (drill 0.3) (layers "F.Cu" "B.Cu") (free yes) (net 4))
 (via (at 96.5 52.2) (size 0.6) (drill 0.3) (layers "F.Cu" "B.Cu") (free yes) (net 4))
 (segment (start 87.39 52.49) (end 86.63 52.49) (width 0.3) (layer "F.Cu") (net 3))
 (segment (start 87.7725 56.85) (end 87.7725 52.8725) (width 0.3) (layer "F.Cu") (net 3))
 (segment (start 87.7725 52.8725) (end 87.39 52.49) (width 0.3) (layer "F.Cu") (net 3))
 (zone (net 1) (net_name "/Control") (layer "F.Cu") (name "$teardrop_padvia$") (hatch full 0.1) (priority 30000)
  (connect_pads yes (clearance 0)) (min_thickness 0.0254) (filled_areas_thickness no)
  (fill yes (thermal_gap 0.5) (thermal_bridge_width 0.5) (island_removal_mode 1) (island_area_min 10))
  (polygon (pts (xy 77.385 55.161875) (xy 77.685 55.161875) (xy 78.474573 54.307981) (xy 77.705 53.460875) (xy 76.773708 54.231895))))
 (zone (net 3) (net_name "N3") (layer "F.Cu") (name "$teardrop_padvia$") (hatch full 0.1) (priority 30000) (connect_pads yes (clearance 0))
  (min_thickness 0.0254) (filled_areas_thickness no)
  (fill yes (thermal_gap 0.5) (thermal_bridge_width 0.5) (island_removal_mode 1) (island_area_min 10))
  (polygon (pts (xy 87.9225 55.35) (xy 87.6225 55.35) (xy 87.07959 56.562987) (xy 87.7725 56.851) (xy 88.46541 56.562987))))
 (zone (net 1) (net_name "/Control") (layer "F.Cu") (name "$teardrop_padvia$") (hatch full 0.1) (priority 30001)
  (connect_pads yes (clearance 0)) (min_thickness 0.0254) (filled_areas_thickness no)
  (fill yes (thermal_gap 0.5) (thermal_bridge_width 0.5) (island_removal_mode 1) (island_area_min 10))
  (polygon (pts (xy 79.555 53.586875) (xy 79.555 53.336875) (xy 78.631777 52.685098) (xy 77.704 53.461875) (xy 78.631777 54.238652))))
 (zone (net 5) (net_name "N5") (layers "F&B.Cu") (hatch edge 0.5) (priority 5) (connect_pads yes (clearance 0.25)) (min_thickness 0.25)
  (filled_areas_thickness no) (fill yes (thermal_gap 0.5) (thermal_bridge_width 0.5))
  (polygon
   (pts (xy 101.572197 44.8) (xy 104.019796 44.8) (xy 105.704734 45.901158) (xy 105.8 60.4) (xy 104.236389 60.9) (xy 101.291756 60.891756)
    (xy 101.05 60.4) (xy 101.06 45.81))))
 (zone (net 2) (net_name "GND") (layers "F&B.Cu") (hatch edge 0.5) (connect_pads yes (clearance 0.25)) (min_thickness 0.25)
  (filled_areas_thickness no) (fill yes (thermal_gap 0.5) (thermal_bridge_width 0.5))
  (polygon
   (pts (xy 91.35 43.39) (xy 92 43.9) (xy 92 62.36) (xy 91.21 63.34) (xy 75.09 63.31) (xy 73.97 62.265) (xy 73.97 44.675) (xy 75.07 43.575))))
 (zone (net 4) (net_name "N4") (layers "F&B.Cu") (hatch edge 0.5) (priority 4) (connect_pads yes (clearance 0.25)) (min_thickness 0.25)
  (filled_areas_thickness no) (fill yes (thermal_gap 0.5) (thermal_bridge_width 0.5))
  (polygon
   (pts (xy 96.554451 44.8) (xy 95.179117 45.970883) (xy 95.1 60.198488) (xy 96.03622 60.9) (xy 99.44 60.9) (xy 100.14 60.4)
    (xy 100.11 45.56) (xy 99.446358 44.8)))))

